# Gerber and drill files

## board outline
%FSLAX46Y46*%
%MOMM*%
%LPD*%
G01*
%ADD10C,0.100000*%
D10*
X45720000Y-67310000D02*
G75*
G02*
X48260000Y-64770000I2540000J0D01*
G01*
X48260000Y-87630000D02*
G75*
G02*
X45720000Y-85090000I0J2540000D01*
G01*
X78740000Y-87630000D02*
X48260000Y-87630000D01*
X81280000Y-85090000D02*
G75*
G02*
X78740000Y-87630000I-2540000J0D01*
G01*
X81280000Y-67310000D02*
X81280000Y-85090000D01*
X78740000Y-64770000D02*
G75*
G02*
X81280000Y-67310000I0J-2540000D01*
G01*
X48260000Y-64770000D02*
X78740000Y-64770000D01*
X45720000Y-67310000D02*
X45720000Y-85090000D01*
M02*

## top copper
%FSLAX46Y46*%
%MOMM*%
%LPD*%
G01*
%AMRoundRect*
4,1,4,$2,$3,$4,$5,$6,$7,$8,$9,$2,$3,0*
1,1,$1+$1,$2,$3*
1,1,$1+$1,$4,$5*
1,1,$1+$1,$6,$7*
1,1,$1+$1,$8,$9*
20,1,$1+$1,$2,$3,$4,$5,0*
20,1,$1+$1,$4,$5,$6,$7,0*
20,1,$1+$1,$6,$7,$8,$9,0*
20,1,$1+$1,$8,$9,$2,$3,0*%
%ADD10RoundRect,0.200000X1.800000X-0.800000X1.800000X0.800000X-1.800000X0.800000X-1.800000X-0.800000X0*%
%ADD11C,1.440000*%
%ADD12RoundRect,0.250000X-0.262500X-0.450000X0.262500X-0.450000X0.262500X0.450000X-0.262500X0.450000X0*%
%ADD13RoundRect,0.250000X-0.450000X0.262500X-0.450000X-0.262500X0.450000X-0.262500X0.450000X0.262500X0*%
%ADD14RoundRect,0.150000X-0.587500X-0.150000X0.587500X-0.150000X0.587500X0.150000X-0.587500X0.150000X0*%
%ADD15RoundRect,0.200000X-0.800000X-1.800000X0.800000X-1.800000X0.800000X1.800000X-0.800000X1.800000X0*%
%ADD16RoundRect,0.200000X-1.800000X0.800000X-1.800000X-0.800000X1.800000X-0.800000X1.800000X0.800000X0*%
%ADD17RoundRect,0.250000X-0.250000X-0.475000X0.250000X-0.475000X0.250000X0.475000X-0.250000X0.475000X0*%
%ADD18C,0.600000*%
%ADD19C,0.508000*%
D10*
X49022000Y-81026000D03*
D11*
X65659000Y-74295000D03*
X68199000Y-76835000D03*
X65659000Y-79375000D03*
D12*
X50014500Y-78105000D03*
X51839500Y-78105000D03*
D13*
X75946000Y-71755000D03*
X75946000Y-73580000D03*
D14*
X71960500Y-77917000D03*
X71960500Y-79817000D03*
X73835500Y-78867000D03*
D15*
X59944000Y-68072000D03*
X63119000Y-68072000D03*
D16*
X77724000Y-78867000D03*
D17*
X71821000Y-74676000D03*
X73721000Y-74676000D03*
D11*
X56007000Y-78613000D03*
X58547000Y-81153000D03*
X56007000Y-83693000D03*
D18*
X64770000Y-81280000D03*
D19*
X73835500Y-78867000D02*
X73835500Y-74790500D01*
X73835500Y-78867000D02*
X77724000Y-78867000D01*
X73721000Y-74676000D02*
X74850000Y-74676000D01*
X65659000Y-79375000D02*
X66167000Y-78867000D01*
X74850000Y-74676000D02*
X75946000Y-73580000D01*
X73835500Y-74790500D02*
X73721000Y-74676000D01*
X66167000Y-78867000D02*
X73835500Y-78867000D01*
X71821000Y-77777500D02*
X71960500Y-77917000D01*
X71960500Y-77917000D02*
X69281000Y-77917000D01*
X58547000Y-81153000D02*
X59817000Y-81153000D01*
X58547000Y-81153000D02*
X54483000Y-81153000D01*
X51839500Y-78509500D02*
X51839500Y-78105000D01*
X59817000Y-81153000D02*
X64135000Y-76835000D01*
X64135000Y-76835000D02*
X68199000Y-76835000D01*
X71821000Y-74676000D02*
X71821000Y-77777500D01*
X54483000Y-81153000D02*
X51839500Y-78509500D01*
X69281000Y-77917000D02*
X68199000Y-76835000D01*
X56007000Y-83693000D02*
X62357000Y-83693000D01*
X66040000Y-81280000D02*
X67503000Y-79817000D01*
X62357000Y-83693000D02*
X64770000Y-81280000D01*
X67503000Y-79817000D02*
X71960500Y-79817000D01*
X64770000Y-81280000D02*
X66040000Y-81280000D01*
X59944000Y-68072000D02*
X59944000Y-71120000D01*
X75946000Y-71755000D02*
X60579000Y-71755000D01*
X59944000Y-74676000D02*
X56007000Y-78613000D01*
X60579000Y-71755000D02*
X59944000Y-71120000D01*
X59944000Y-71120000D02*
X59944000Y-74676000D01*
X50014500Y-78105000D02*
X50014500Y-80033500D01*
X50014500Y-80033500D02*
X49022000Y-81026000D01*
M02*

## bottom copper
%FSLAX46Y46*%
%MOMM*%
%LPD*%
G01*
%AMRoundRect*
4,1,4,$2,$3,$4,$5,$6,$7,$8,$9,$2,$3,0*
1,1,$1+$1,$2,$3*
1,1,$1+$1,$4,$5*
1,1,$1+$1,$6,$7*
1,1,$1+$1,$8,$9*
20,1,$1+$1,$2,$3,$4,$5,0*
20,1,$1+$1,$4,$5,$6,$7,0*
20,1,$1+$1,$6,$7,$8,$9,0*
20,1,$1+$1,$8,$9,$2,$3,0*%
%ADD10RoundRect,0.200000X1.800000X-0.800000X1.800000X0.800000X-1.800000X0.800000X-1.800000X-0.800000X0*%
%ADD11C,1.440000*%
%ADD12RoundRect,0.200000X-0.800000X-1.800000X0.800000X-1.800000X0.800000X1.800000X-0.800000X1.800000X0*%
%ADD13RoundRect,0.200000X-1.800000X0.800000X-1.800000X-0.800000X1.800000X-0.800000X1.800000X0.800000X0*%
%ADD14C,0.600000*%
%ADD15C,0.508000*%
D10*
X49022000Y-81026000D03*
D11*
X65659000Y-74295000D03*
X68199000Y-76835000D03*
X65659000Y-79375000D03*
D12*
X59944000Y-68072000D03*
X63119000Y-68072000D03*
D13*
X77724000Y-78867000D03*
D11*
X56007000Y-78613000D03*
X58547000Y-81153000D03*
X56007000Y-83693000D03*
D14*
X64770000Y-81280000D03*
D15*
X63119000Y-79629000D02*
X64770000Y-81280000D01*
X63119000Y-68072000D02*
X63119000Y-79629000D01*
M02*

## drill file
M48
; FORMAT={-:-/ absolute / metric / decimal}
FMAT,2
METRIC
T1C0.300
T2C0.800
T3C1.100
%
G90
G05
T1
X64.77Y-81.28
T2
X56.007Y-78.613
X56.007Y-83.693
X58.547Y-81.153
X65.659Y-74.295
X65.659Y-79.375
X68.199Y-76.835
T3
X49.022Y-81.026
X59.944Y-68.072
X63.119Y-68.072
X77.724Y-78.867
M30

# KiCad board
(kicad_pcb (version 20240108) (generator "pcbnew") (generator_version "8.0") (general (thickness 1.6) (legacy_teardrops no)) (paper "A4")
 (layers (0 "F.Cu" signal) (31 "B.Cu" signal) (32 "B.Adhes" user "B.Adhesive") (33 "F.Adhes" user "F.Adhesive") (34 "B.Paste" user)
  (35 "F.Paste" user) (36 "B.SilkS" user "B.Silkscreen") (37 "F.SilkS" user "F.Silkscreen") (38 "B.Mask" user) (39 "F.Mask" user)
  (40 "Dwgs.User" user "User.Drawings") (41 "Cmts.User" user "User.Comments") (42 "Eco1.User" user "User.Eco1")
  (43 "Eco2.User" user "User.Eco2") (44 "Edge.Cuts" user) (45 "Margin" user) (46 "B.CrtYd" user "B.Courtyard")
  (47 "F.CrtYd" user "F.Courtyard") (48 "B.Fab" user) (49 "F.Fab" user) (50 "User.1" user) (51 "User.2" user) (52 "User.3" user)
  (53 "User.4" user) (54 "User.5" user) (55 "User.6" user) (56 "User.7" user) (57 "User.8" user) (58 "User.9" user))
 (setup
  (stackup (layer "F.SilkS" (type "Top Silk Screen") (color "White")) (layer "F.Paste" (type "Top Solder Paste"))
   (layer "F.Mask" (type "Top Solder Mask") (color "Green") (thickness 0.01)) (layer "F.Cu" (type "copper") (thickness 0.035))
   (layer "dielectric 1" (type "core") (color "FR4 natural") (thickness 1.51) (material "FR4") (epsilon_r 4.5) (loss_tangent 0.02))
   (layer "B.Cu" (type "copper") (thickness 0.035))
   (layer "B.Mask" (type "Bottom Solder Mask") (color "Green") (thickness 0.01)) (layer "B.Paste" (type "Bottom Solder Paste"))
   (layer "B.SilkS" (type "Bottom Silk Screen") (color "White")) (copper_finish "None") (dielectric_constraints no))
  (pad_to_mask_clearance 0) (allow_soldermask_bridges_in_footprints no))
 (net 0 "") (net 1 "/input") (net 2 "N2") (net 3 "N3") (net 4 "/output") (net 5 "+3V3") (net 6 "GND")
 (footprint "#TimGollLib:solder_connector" (layer "F.Cu") (at 49.022 81.026 90)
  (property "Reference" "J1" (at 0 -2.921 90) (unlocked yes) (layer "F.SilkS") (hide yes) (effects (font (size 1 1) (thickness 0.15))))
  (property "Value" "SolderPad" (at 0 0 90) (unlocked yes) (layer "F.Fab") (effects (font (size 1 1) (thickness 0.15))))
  (pad "1" thru_hole roundrect (at 0 0 90) (size 2 4) (drill 1.1) (layers "*.Cu" "*.Mask") (remove_unused_layers no) (roundrect_rratio 0.1)
   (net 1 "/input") (solder_mask_margin 0.102)))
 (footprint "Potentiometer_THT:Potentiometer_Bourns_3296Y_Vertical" (layer "F.Cu") (at 65.659 74.295 90)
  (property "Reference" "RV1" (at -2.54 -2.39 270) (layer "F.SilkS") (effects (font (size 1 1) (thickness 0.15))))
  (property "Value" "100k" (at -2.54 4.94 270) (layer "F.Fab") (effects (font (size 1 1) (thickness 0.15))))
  (pad "1" thru_hole circle (at 0 0 90) (size 1.44 1.44) (drill 0.8) (layers "*.Cu" "*.Mask") (remove_unused_layers no) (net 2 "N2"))
  (pad "2" thru_hole circle (at -2.54 2.54 90) (size 1.44 1.44) (drill 0.8) (layers "*.Cu" "*.Mask") (remove_unused_layers no) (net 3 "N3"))
  (pad "3" thru_hole circle (at -5.08 0 90) (size 1.44 1.44) (drill 0.8) (layers "*.Cu" "*.Mask") (remove_unused_layers no)
   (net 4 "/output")))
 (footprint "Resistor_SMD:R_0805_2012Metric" (layer "F.Cu") (at 50.927 78.105)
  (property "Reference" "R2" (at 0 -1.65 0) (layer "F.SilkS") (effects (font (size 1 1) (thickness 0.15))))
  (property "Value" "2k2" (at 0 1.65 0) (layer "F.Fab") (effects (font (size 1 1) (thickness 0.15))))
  (pad "1" smd roundrect (at -0.9125 0) (size 1.025 1.4) (layers "F.Cu" "F.Paste" "F.Mask") (roundrect_rratio 0.243902) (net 1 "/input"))
  (pad "2" smd roundrect (at 0.9125 0) (size 1.025 1.4) (layers "F.Cu" "F.Paste" "F.Mask") (roundrect_rratio 0.243902) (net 3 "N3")))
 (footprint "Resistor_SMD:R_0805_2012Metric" (layer "F.Cu") (at 75.946 72.6675 -90)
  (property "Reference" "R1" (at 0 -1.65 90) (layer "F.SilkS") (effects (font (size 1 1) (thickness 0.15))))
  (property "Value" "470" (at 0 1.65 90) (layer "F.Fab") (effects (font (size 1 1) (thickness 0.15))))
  (pad "1" smd roundrect (at -0.9125 0 270) (size 1.025 1.4) (layers "F.Cu" "F.Paste" "F.Mask") (roundrect_rratio 0.243902) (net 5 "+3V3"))
  (pad "2" smd roundrect (at 0.9125 0 270) (size 1.025 1.4) (layers "F.Cu" "F.Paste" "F.Mask") (roundrect_rratio 0.243902) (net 4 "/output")))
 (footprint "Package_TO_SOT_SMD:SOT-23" (layer "F.Cu") (at 72.898 78.867)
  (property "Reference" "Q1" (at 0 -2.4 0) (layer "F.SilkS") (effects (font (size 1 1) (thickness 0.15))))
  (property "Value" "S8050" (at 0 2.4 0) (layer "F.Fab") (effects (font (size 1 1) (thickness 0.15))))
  (pad "1" smd roundrect (at -0.9375 -0.95) (size 1.475 0.6) (layers "F.Cu" "F.Paste" "F.Mask") (roundrect_rratio 0.25) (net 3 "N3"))
  (pad "2" smd roundrect (at -0.9375 0.95) (size 1.475 0.6) (layers "F.Cu" "F.Paste" "F.Mask") (roundrect_rratio 0.25) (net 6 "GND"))
  (pad "3" smd roundrect (at 0.9375 0) (size 1.475 0.6) (layers "F.Cu" "F.Paste" "F.Mask") (roundrect_rratio 0.25) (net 4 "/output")))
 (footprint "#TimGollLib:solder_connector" (layer "F.Cu") (at 59.944 68.072)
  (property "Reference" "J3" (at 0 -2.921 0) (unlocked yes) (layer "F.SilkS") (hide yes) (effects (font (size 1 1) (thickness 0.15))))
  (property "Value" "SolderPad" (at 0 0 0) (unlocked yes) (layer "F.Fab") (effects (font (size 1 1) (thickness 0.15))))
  (pad "1" thru_hole roundrect (at 0 0) (size 2 4) (drill 1.1) (layers "*.Cu" "*.Mask") (remove_unused_layers no) (roundrect_rratio 0.1)
   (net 5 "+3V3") (solder_mask_margin 0.102)))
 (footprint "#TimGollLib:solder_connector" (layer "F.Cu") (at 63.119 68.072)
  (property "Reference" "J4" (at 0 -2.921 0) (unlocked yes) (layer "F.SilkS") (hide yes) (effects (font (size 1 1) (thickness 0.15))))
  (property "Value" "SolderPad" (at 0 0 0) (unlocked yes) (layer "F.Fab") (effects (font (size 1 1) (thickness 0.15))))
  (pad "1" thru_hole roundrect (at 0 0) (size 2 4) (drill 1.1) (layers "*.Cu" "*.Mask") (remove_unused_layers no) (roundrect_rratio 0.1)
   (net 6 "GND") (solder_mask_margin 0.102)))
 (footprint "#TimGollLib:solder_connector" (layer "F.Cu") (at 77.724 78.867 -90)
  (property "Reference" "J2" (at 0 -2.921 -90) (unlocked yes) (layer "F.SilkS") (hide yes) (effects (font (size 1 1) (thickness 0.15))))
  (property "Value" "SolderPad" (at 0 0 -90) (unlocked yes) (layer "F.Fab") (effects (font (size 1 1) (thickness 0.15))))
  (pad "1" thru_hole roundrect (at 0 0 270) (size 2 4) (drill 1.1) (layers "*.Cu" "*.Mask") (remove_unused_layers no) (roundrect_rratio 0.1)
   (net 4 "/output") (solder_mask_margin 0.102)))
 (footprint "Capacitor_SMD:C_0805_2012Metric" (layer "F.Cu") (at 72.771 74.676)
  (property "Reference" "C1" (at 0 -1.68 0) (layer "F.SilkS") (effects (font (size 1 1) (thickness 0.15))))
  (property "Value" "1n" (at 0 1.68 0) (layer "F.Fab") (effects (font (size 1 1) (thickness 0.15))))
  (pad "1" smd roundrect (at -0.95 0) (size 1 1.45) (layers "F.Cu" "F.Paste" "F.Mask") (roundrect_rratio 0.25) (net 3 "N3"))
  (pad "2" smd roundrect (at 0.95 0) (size 1 1.45) (layers "F.Cu" "F.Paste" "F.Mask") (roundrect_rratio 0.25) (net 4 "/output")))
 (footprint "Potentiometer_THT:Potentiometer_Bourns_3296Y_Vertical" (layer "F.Cu") (at 56.007 78.613 90)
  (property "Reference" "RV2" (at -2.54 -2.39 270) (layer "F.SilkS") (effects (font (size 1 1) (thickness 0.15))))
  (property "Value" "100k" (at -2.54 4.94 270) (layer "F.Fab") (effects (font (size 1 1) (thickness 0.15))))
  (pad "1" thru_hole circle (at 0 0 90) (size 1.44 1.44) (drill 0.8) (layers "*.Cu" "*.Mask") (remove_unused_layers no) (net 5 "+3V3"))
  (pad "2" thru_hole circle (at -2.54 2.54 90) (size 1.44 1.44) (drill 0.8) (layers "*.Cu" "*.Mask") (remove_unused_layers no) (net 3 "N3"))
  (pad "3" thru_hole circle (at -5.08 0 90) (size 1.44 1.44) (drill 0.8) (layers "*.Cu" "*.Mask") (remove_unused_layers no) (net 6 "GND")))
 (gr_arc (start 45.72 67.31) (mid 46.463949 65.513949) (end 48.26 64.77) (stroke (width 0.1) (type default)) (layer "Edge.Cuts"))
 (gr_arc (start 48.26 87.63) (mid 46.463949 86.886051) (end 45.72 85.09) (stroke (width 0.1) (type default)) (layer "Edge.Cuts"))
 (gr_line (start 78.74 87.63) (end 48.26 87.63) (stroke (width 0.1) (type default)) (layer "Edge.Cuts"))
 (gr_arc (start 81.28 85.09) (mid 80.536051 86.886051) (end 78.74 87.63) (stroke (width 0.1) (type default)) (layer "Edge.Cuts"))
 (gr_line (start 81.28 67.31) (end 81.28 85.09) (stroke (width 0.1) (type default)) (layer "Edge.Cuts"))
 (gr_arc (start 78.74 64.77) (mid 80.536051 65.513949) (end 81.28 67.31) (stroke (width 0.1) (type default)) (layer "Edge.Cuts"))
 (gr_line (start 48.26 64.77) (end 78.74 64.77) (stroke (width 0.1) (type default)) (layer "Edge.Cuts"))
 (gr_line (start 45.72 67.31) (end 45.72 85.09) (stroke (width 0.1) (type default)) (layer "Edge.Cuts"))
 (segment (start 73.8355 78.867) (end 73.8355 74.7905) (width 0.508) (layer "F.Cu") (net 4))
 (segment (start 73.8355 78.867) (end 77.724 78.867) (width 0.508) (layer "F.Cu") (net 4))
 (segment (start 73.721 74.676) (end 74.85 74.676) (width 0.508) (layer "F.Cu") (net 4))
 (segment (start 65.659 79.375) (end 66.167 78.867) (width 0.508) (layer "F.Cu") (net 4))
 (segment (start 74.85 74.676) (end 75.946 73.58) (width 0.508) (layer "F.Cu") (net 4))
 (segment (start 73.8355 74.7905) (end 73.721 74.676) (width 0.508) (layer "F.Cu") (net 4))
 (segment (start 66.167 78.867) (end 73.8355 78.867) (width 0.508) (layer "F.Cu") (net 4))
 (segment (start 71.821 77.7775) (end 71.9605 77.917) (width 0.508) (layer "F.Cu") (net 3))
 (segment (start 71.9605 77.917) (end 69.281 77.917) (width 0.508) (layer "F.Cu") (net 3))
 (segment (start 58.547 81.153) (end 59.817 81.153) (width 0.508) (layer "F.Cu") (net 3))
 (segment (start 58.547 81.153) (end 54.483 81.153) (width 0.508) (layer "F.Cu") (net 3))
 (segment (start 51.8395 78.5095) (end 51.8395 78.105) (width 0.508) (layer "F.Cu") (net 3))
 (segment (start 59.817 81.153) (end 64.135 76.835) (width 0.508) (layer "F.Cu") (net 3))
 (segment (start 64.135 76.835) (end 68.199 76.835) (width 0.508) (layer "F.Cu") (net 3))
 (segment (start 71.821 74.676) (end 71.821 77.7775) (width 0.508) (layer "F.Cu") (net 3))
 (segment (start 54.483 81.153) (end 51.8395 78.5095) (width 0.508) (layer "F.Cu") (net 3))
 (segment (start 69.281 77.917) (end 68.199 76.835) (width 0.508) (layer "F.Cu") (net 3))
 (segment (start 56.007 83.693) (end 62.357 83.693) (width 0.508) (layer "F.Cu") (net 6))
 (segment (start 66.04 81.28) (end 67.503 79.817) (width 0.508) (layer "F.Cu") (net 6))
 (segment (start 62.357 83.693) (end 64.77 81.28) (width 0.508) (layer "F.Cu") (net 6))
 (segment (start 67.503 79.817) (end 71.9605 79.817) (width 0.508) (layer "F.Cu") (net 6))
 (segment (start 64.77 81.28) (end 66.04 81.28) (width 0.508) (layer "F.Cu") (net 6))
 (via (at 64.77 81.28) (size 0.6) (drill 0.3) (layers "F.Cu" "B.Cu") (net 6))
 (segment (start 63.119 79.629) (end 64.77 81.28) (width 0.508) (layer "B.Cu") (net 6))
 (segment (start 63.119 68.072) (end 63.119 79.629) (width 0.508) (layer "B.Cu") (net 6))
 (segment (start 59.944 68.072) (end 59.944 71.12) (width 0.508) (layer "F.Cu") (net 5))
 (segment (start 75.946 71.755) (end 60.579 71.755) (width 0.508) (layer "F.Cu") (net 5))
 (segment (start 59.944 74.676) (end 56.007 78.613) (width 0.508) (layer "F.Cu") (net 5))
 (segment (start 60.579 71.755) (end 59.944 71.12) (width 0.508) (layer "F.Cu") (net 5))
 (segment (start 59.944 71.12) (end 59.944 74.676) (width 0.508) (layer "F.Cu") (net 5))
 (segment (start 50.0145 78.105) (end 50.0145 80.0335) (width 0.508) (layer "F.Cu") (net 1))
 (segment (start 50.0145 80.0335) (end 49.022 81.026) (width 0.508) (layer "F.Cu") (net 1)))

